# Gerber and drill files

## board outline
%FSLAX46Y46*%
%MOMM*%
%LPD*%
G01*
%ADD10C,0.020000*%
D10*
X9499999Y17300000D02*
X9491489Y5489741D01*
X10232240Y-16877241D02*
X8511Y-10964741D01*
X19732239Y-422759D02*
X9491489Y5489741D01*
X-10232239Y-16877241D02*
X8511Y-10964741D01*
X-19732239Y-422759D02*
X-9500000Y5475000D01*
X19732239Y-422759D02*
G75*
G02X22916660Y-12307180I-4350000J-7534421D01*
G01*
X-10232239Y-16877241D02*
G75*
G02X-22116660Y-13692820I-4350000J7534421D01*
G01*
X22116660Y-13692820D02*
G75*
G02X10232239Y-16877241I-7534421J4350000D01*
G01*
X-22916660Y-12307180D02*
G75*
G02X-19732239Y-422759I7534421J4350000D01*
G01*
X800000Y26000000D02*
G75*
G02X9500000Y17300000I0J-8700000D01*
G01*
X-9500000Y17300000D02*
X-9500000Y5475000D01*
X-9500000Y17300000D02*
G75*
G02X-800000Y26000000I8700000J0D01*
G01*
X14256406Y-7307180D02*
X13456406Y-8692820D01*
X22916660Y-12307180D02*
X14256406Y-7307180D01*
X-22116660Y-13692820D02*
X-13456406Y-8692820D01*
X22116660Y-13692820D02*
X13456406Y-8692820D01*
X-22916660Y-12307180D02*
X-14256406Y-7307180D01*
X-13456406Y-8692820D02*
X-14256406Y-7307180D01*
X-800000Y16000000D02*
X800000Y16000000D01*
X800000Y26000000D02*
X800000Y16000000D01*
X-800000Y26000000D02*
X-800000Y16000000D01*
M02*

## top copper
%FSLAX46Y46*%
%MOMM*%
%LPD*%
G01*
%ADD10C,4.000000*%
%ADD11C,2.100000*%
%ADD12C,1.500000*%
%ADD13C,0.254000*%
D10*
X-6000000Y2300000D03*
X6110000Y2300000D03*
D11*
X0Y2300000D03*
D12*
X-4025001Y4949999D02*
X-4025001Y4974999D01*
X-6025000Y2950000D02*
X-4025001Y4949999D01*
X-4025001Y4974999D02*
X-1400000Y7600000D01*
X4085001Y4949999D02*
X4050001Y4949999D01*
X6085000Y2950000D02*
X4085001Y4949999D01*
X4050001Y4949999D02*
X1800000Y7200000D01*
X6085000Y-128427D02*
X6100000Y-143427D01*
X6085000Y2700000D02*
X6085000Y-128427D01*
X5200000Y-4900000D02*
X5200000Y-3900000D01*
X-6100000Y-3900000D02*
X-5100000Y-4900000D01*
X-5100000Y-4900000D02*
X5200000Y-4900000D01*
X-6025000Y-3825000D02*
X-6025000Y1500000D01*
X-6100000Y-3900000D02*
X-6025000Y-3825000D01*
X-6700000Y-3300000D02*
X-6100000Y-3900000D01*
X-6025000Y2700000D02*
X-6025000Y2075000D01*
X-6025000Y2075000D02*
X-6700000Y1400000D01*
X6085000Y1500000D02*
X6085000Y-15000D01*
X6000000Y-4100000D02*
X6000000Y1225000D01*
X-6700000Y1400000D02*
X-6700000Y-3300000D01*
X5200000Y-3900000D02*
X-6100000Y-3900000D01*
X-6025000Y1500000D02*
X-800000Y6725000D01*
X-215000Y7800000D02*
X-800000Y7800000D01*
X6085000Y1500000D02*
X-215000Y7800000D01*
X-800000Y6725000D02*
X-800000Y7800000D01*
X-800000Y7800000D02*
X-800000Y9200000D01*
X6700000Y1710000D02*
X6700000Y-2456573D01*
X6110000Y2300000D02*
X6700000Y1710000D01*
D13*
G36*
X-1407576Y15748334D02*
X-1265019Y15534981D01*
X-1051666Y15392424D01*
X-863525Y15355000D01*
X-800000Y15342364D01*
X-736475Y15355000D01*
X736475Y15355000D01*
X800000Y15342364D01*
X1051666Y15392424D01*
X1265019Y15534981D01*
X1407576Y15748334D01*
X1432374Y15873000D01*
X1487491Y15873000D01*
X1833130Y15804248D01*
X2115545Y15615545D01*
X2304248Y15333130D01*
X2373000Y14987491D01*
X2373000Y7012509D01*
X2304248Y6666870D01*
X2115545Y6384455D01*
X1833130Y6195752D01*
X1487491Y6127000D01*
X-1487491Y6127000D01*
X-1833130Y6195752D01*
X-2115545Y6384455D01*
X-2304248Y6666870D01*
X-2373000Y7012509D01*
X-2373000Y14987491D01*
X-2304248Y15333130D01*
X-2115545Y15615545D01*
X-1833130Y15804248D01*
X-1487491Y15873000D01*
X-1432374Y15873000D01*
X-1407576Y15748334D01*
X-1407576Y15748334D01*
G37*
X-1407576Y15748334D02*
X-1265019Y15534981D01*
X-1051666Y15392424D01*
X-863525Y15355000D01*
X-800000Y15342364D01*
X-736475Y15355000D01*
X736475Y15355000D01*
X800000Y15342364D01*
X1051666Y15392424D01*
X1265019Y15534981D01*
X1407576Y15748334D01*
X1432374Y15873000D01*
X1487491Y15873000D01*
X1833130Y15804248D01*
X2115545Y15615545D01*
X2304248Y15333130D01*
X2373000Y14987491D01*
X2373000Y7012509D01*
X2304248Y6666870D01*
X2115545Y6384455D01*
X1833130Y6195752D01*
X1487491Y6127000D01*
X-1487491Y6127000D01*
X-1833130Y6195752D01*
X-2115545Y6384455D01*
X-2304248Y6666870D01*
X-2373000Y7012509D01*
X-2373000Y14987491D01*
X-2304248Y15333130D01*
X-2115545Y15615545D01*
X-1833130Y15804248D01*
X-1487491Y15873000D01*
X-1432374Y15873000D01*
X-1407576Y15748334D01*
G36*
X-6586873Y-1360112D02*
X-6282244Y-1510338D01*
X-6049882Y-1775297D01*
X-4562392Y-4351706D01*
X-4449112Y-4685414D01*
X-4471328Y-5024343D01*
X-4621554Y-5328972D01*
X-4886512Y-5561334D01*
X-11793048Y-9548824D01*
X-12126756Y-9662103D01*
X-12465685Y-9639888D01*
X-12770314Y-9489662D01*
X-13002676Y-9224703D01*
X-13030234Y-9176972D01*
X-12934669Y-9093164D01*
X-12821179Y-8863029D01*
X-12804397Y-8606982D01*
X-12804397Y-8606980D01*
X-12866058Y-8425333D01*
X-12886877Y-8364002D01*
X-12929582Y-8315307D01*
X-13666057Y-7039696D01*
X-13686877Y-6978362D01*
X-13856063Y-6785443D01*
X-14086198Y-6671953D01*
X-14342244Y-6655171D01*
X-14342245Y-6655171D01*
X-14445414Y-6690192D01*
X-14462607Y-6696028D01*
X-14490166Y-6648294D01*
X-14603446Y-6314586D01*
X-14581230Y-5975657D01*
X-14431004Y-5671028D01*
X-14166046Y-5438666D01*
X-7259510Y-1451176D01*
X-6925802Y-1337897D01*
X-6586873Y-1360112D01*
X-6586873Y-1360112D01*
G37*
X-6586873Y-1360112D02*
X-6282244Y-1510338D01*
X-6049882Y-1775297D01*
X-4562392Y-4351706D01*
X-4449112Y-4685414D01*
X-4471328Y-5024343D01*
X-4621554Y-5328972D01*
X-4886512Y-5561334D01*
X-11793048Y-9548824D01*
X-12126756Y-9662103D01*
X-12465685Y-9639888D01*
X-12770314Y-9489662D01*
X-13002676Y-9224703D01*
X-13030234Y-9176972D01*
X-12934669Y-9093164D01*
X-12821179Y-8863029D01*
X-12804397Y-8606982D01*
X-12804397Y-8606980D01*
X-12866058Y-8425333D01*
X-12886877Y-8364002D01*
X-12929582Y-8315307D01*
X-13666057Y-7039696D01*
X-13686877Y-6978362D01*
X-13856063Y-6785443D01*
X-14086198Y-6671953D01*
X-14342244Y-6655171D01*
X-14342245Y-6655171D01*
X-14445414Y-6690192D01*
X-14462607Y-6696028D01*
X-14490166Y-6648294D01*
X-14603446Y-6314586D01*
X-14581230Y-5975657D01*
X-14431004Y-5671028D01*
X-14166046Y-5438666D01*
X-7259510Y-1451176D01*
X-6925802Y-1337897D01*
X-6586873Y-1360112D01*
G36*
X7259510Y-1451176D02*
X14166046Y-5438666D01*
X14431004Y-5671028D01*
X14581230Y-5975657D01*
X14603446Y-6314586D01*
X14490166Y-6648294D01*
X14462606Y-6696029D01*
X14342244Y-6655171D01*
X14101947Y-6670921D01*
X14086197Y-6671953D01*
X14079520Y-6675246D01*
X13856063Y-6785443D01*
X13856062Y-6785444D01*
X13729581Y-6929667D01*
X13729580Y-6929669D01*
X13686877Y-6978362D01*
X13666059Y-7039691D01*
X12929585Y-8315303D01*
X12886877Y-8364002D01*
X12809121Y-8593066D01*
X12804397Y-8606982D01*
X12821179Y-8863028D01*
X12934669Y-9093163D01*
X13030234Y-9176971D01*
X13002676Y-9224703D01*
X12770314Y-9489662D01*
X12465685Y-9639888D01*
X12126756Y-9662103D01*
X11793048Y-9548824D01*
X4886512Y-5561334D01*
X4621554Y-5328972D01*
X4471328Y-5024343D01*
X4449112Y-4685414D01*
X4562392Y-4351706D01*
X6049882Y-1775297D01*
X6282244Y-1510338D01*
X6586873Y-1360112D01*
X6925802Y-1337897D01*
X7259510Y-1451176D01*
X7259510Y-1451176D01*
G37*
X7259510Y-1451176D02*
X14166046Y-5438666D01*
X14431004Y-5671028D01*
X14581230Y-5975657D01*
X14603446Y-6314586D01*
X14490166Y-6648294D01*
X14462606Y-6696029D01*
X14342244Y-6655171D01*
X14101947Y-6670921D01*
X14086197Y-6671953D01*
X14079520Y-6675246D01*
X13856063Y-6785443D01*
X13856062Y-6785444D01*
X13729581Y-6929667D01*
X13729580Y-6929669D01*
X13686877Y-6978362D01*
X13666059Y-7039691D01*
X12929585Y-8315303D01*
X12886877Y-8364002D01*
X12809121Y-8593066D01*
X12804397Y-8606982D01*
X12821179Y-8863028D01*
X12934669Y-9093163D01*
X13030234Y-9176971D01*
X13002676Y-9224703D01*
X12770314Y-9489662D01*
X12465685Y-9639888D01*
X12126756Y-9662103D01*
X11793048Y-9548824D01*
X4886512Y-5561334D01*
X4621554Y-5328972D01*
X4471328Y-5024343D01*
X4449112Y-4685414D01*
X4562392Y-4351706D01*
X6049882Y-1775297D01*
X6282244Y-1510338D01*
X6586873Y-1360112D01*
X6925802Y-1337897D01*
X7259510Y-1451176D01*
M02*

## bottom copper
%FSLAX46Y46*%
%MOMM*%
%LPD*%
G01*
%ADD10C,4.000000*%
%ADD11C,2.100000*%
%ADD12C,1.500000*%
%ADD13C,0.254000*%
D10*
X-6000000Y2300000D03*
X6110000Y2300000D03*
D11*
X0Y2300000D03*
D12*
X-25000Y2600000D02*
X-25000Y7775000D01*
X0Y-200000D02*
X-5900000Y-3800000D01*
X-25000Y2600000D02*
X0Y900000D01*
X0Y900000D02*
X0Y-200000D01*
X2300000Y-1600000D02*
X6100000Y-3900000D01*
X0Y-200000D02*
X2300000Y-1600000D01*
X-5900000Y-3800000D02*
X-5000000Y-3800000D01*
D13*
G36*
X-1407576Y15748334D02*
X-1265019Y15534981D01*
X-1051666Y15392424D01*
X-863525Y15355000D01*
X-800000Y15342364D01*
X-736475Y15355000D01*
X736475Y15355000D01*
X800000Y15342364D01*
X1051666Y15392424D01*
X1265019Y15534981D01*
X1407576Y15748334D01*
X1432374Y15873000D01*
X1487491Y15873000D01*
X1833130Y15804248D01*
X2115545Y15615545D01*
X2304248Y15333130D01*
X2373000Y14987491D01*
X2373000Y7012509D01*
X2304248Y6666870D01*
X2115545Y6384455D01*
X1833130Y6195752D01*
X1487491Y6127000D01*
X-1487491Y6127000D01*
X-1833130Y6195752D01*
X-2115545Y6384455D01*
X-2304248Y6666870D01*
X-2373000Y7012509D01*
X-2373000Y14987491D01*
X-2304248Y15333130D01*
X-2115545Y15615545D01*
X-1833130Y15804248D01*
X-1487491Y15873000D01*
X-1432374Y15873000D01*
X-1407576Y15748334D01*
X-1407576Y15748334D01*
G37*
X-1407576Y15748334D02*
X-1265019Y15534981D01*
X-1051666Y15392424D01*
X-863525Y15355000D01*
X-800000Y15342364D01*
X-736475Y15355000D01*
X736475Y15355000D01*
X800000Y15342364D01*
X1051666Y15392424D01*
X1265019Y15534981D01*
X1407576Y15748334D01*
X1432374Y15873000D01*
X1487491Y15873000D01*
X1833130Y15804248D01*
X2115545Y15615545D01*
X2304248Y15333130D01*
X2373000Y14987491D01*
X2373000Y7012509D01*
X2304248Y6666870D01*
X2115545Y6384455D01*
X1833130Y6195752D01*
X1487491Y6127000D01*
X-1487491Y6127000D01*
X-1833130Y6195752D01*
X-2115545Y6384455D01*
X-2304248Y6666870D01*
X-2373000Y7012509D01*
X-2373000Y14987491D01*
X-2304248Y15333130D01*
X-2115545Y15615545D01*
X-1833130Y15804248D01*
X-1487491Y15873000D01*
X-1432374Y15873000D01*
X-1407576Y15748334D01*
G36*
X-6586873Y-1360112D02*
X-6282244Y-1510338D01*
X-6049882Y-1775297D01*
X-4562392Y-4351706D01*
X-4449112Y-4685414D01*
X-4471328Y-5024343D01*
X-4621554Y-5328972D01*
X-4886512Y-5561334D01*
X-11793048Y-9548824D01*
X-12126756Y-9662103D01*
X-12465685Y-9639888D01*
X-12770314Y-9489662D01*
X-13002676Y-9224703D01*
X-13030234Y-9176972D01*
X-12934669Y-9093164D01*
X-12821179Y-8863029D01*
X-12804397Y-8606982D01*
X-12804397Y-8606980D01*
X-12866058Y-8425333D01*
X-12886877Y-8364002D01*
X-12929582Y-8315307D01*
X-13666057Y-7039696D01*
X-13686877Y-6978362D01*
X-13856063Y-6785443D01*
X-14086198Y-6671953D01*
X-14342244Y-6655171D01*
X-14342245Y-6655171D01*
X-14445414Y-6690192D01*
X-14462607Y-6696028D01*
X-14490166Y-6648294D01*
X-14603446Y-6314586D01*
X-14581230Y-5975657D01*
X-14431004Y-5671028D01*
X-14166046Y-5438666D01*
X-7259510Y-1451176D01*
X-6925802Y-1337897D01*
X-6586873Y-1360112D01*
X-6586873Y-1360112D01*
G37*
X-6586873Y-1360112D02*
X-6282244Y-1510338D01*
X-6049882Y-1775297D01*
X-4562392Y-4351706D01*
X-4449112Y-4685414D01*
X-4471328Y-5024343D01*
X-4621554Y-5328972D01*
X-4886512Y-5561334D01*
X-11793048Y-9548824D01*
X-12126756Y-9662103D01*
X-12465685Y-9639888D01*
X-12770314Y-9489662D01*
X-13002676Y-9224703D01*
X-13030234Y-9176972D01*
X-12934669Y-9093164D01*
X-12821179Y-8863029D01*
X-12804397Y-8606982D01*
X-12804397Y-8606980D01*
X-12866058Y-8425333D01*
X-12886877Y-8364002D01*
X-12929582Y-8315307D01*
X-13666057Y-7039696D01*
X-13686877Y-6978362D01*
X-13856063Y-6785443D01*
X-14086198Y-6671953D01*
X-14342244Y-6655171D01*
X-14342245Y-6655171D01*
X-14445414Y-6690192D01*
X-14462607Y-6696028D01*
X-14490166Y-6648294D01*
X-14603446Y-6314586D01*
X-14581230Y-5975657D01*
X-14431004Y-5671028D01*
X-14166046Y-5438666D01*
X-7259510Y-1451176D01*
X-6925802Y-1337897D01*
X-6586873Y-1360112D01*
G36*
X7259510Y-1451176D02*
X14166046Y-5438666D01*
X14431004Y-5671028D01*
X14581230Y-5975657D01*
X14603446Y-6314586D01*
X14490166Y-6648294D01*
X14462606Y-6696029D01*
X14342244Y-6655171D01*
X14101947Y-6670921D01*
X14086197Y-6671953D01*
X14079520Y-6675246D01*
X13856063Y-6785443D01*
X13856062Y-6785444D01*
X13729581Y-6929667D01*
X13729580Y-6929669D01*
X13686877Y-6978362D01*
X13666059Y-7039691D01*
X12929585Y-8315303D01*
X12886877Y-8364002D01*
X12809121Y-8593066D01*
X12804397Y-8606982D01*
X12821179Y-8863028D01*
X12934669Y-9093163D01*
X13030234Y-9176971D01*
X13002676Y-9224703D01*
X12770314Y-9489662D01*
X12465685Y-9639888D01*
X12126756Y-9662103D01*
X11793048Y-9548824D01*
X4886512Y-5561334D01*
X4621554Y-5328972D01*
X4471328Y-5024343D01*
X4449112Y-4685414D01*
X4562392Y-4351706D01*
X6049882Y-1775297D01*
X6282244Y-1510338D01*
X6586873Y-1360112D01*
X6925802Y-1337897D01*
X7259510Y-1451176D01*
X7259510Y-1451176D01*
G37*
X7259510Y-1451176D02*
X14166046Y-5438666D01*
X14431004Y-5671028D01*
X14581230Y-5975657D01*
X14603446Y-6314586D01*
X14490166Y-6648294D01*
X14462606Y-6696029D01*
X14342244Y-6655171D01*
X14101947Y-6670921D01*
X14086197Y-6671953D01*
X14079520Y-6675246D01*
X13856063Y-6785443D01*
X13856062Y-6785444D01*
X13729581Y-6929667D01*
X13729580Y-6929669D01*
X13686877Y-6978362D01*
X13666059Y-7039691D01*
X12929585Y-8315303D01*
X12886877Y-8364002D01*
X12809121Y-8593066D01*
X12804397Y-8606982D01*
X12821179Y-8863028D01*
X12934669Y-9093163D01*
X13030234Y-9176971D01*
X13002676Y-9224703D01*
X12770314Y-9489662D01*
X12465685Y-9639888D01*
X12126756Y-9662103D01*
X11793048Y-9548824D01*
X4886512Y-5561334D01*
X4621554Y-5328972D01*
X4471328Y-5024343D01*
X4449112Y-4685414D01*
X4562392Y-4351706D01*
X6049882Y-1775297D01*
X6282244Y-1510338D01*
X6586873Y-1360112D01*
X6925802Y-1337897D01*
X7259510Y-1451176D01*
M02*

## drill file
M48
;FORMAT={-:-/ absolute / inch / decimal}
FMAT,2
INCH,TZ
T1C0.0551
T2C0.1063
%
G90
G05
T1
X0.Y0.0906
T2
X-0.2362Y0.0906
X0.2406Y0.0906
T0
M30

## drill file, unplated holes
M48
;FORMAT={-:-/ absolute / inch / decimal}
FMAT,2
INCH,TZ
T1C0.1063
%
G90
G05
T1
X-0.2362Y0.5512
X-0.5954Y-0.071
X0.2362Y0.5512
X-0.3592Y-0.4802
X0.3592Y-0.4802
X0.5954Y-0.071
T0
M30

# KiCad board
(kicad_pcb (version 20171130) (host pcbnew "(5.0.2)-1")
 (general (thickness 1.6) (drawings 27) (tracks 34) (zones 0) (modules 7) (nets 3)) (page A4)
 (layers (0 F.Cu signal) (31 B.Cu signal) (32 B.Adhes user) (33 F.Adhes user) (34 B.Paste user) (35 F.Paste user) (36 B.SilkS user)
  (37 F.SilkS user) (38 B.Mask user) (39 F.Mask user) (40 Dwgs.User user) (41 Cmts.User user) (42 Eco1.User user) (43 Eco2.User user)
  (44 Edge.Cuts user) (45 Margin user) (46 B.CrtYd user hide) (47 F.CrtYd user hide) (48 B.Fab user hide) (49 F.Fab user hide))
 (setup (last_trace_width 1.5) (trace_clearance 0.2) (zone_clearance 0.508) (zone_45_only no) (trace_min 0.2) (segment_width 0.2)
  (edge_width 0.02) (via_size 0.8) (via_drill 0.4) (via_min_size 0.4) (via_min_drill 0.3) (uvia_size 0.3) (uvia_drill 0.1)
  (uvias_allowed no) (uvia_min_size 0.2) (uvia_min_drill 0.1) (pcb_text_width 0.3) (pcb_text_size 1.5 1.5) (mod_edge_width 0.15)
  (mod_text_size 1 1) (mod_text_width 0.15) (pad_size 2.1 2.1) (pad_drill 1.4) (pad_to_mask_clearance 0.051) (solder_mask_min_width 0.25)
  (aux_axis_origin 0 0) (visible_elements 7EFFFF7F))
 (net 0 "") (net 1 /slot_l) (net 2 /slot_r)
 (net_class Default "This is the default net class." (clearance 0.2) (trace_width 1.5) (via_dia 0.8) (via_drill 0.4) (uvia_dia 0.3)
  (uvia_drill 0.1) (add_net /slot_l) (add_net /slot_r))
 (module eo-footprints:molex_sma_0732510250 (layer F.Cu) (at 0 -2.3)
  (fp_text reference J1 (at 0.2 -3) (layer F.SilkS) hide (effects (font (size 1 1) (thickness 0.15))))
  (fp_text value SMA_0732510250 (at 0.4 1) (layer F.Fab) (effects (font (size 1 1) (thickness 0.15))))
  (pad 2 thru_hole circle (at -6 0) (size 4 4) (drill 2.7) (layers *.Cu *.Mask) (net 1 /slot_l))
  (pad 2 thru_hole circle (at 6.11 0) (size 4 4) (drill 2.7) (layers *.Cu *.Mask) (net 1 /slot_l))
  (pad 1 thru_hole circle (at 0 0) (size 2.1 2.1) (drill 1.4) (layers *.Cu *.Mask) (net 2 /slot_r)))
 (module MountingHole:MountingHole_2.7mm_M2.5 (layer F.Cu) (at 15.124356 1.803848 240)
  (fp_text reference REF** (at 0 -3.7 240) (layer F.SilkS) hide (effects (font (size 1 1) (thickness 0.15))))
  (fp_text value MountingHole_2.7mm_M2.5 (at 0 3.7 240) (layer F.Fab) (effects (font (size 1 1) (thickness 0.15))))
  (pad 1 np_thru_hole circle (at 0 0 240) (size 2.7 2.7) (drill 2.7) (layers *.Cu *.Mask)))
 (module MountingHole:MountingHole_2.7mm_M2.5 (layer F.Cu) (at -9.124356 12.196152 120)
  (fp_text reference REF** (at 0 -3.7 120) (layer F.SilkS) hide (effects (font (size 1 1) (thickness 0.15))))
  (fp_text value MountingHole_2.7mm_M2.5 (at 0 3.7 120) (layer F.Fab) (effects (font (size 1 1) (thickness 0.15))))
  (pad 1 np_thru_hole circle (at 0 0 120) (size 2.7 2.7) (drill 2.7) (layers *.Cu *.Mask)))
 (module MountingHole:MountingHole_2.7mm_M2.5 (layer F.Cu) (at 9.124356 12.196152 240)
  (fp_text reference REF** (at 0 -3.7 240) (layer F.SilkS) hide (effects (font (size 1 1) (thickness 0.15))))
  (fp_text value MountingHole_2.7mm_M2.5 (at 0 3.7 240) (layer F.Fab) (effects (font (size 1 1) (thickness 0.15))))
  (pad 1 np_thru_hole circle (at 0 0 240) (size 2.7 2.7) (drill 2.7) (layers *.Cu *.Mask)))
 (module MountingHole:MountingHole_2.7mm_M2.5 (layer F.Cu) (at -15.124356 1.803848 120)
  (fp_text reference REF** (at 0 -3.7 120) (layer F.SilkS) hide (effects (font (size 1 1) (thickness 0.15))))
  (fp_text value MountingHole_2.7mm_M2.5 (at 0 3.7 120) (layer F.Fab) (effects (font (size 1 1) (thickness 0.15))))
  (pad 1 np_thru_hole circle (at 0 0 120) (size 2.7 2.7) (drill 2.7) (layers *.Cu *.Mask)))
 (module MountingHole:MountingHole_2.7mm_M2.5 (layer F.Cu) (at 6 -14)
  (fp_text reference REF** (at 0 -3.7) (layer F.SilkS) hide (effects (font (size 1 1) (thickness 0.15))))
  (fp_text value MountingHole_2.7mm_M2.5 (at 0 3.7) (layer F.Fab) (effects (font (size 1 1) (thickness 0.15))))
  (pad 1 np_thru_hole circle (at 0 0) (size 2.7 2.7) (drill 2.7) (layers *.Cu *.Mask)))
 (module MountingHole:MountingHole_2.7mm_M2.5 (layer F.Cu) (at -6 -14)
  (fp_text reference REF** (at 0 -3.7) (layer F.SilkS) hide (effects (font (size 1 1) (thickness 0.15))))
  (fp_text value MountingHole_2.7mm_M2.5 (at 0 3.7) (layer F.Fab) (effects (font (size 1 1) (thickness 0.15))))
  (pad 1 np_thru_hole circle (at 0 0) (size 2.7 2.7) (drill 2.7) (layers *.Cu *.Mask)))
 (gr_line (start 9.499999 -17.3) (end 9.491489 -5.489741) (layer Edge.Cuts) (width 0.02))
 (gr_line (start 10.23224 16.877241) (end 0.008511 10.964741) (layer Edge.Cuts) (width 0.02))
 (gr_line (start 19.732239 0.422759) (end 9.491489 -5.489741) (layer Edge.Cuts) (width 0.02))
 (gr_line (start -10.232239 16.877241) (end 0.008511 10.964741) (layer Edge.Cuts) (width 0.02))
 (gr_line (start -19.732239 0.422759) (end -9.5 -5.475) (layer Edge.Cuts) (width 0.02))
 (gr_arc (start 15.382239 7.95718) (end 22.91666 12.30718) (angle -90) (layer Edge.Cuts) (width 0.02))
 (gr_arc (start -14.582239 9.34282) (end -22.11666 13.69282) (angle -90) (layer Edge.Cuts) (width 0.02))
 (gr_arc (start 14.582239 9.34282) (end 10.232239 16.877241) (angle -90) (layer Edge.Cuts) (width 0.02))
 (gr_arc (start -15.382239 7.95718) (end -19.732239 0.422759) (angle -90) (layer Edge.Cuts) (width 0.02))
 (gr_arc (start 0.8 -17.3) (end 9.5 -17.3) (angle -90) (layer Edge.Cuts) (width 0.02))
 (gr_line (start -9.5 -17.3) (end -9.5 -5.475) (layer Edge.Cuts) (width 0.02))
 (gr_arc (start -0.8 -17.3) (end -0.8 -26) (angle -90) (layer Edge.Cuts) (width 0.02))
 (gr_line (start 14.256406 7.30718) (end 13.456406 8.69282) (layer Edge.Cuts) (width 0.02))
 (gr_line (start 22.91666 12.30718) (end 14.256406 7.30718) (layer Edge.Cuts) (width 0.02))
 (gr_line (start -22.11666 13.69282) (end -13.456406 8.69282) (layer Edge.Cuts) (width 0.02))
 (gr_line (start 22.11666 13.69282) (end 13.456406 8.69282) (layer Edge.Cuts) (width 0.02))
 (gr_line (start -22.91666 12.30718) (end -14.256406 7.30718) (layer Edge.Cuts) (width 0.02))
 (gr_line (start -13.456406 8.69282) (end -14.256406 7.30718) (layer Edge.Cuts) (width 0.02))
 (gr_line (start -0.8 -16) (end 0.8 -16) (layer Edge.Cuts) (width 0.02))
 (gr_line (start 0.8 -26) (end 0.8 -16) (layer Edge.Cuts) (width 0.02))
 (gr_line (start -0.8 -26) (end -0.8 -16) (layer Edge.Cuts) (width 0.02))
 (segment (start -0.025 -2.6) (end -0.025 -7.775) (width 1.5) (layer B.Cu) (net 2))
 (segment (start 0 0.2) (end -5.9 3.8) (width 1.5) (layer B.Cu) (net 2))
 (segment (start -0.025 -2.6) (end 0 -0.9) (width 1.5) (layer B.Cu) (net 2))
 (segment (start 0 -0.9) (end 0 0.2) (width 1.5) (layer B.Cu) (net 2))
 (segment (start 2.3 1.6) (end 6.1 3.9) (width 1.5) (layer B.Cu) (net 2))
 (segment (start 0 0.2) (end 2.3 1.6) (width 1.5) (layer B.Cu) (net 2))
 (segment (start -5.9 3.8) (end -5 3.8) (width 1.5) (layer B.Cu) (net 2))
 (segment (start -4.025001 -4.949999) (end -4.025001 -4.974999) (width 1.5) (layer F.Cu) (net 1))
 (segment (start -6.025 -2.95) (end -4.025001 -4.949999) (width 1.5) (layer F.Cu) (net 1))
 (segment (start -4.025001 -4.974999) (end -1.4 -7.6) (width 1.5) (layer F.Cu) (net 1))
 (segment (start 4.085001 -4.949999) (end 4.050001 -4.949999) (width 1.5) (layer F.Cu) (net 1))
 (segment (start 6.085 -2.95) (end 4.085001 -4.949999) (width 1.5) (layer F.Cu) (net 1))
 (segment (start 4.050001 -4.949999) (end 1.8 -7.2) (width 1.5) (layer F.Cu) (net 1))
 (segment (start 6.085 0.128427) (end 6.1 0.143427) (width 1.5) (layer F.Cu) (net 1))
 (segment (start 6.085 -2.7) (end 6.085 0.128427) (width 1.5) (layer F.Cu) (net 1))
 (segment (start 5.2 4.9) (end 5.2 3.9) (width 1.5) (layer F.Cu) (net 1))
 (segment (start -6.1 3.9) (end -5.1 4.9) (width 1.5) (layer F.Cu) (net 1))
 (segment (start -5.1 4.9) (end 5.2 4.9) (width 1.5) (layer F.Cu) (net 1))
 (segment (start -6.025 3.825) (end -6.025 -1.5) (width 1.5) (layer F.Cu) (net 1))
 (segment (start -6.1 3.9) (end -6.025 3.825) (width 1.5) (layer F.Cu) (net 1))
 (segment (start -6.7 3.3) (end -6.1 3.9) (width 1.5) (layer F.Cu) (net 1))
 (segment (start -6.025 -2.7) (end -6.025 -2.075) (width 1.5) (layer F.Cu) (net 1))
 (segment (start -6.025 -2.075) (end -6.7 -1.4) (width 1.5) (layer F.Cu) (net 1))
 (segment (start 6.085 -1.5) (end 6.085 0.015) (width 1.5) (layer F.Cu) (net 1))
 (segment (start 6 4.1) (end 6 -1.225) (width 1.5) (layer F.Cu) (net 1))
 (segment (start -6.7 -1.4) (end -6.7 3.3) (width 1.5) (layer F.Cu) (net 1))
 (segment (start 5.2 3.9) (end -6.1 3.9) (width 1.5) (layer F.Cu) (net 1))
 (segment (start -6.025 -1.5) (end -0.8 -6.725) (width 1.5) (layer F.Cu) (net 1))
 (segment (start -0.215 -7.8) (end -0.8 -7.8) (width 1.5) (layer F.Cu) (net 1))
 (segment (start 6.085 -1.5) (end -0.215 -7.8) (width 1.5) (layer F.Cu) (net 1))
 (segment (start -0.8 -6.725) (end -0.8 -7.8) (width 1.5) (layer F.Cu) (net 1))
 (segment (start -0.8 -7.8) (end -0.8 -9.2) (width 1.5) (layer F.Cu) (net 1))
 (segment (start 6.7 -1.71) (end 6.7 2.456573) (width 1.5) (layer F.Cu) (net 1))
 (segment (start 6.11 -2.3) (end 6.7 -1.71) (width 1.5) (layer F.Cu) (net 1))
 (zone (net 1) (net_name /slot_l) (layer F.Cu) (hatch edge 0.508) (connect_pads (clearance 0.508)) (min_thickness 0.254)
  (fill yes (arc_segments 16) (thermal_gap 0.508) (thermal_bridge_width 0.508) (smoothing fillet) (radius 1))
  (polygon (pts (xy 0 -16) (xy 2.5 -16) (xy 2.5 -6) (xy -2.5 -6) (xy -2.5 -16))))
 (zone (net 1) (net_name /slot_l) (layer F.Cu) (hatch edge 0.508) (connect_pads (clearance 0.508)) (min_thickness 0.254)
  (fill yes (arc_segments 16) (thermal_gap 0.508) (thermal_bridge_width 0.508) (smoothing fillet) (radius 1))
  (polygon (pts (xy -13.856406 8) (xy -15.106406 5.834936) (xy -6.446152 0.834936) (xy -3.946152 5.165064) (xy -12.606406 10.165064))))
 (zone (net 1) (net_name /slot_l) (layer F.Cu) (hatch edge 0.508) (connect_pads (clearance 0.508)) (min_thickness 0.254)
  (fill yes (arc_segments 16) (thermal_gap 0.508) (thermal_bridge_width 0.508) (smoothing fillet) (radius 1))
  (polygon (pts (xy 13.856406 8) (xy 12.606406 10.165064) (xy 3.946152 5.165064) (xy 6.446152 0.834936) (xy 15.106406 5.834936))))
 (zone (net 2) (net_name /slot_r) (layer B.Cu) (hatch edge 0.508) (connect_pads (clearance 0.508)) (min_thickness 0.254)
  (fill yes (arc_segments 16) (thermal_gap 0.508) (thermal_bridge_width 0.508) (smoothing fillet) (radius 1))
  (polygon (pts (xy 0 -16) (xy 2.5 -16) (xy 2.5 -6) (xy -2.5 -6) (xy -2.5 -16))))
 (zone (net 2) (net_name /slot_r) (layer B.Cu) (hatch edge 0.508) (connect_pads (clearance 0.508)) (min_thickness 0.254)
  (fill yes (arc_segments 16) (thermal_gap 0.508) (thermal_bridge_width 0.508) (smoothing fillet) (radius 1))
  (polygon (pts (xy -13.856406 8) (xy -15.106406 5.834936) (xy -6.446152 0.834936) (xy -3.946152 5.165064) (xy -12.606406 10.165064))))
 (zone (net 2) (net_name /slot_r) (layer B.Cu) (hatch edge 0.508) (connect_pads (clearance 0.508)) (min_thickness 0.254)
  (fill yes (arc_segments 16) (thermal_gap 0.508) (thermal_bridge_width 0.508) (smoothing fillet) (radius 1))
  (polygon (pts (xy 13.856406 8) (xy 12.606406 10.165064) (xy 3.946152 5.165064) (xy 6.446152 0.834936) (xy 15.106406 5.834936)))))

